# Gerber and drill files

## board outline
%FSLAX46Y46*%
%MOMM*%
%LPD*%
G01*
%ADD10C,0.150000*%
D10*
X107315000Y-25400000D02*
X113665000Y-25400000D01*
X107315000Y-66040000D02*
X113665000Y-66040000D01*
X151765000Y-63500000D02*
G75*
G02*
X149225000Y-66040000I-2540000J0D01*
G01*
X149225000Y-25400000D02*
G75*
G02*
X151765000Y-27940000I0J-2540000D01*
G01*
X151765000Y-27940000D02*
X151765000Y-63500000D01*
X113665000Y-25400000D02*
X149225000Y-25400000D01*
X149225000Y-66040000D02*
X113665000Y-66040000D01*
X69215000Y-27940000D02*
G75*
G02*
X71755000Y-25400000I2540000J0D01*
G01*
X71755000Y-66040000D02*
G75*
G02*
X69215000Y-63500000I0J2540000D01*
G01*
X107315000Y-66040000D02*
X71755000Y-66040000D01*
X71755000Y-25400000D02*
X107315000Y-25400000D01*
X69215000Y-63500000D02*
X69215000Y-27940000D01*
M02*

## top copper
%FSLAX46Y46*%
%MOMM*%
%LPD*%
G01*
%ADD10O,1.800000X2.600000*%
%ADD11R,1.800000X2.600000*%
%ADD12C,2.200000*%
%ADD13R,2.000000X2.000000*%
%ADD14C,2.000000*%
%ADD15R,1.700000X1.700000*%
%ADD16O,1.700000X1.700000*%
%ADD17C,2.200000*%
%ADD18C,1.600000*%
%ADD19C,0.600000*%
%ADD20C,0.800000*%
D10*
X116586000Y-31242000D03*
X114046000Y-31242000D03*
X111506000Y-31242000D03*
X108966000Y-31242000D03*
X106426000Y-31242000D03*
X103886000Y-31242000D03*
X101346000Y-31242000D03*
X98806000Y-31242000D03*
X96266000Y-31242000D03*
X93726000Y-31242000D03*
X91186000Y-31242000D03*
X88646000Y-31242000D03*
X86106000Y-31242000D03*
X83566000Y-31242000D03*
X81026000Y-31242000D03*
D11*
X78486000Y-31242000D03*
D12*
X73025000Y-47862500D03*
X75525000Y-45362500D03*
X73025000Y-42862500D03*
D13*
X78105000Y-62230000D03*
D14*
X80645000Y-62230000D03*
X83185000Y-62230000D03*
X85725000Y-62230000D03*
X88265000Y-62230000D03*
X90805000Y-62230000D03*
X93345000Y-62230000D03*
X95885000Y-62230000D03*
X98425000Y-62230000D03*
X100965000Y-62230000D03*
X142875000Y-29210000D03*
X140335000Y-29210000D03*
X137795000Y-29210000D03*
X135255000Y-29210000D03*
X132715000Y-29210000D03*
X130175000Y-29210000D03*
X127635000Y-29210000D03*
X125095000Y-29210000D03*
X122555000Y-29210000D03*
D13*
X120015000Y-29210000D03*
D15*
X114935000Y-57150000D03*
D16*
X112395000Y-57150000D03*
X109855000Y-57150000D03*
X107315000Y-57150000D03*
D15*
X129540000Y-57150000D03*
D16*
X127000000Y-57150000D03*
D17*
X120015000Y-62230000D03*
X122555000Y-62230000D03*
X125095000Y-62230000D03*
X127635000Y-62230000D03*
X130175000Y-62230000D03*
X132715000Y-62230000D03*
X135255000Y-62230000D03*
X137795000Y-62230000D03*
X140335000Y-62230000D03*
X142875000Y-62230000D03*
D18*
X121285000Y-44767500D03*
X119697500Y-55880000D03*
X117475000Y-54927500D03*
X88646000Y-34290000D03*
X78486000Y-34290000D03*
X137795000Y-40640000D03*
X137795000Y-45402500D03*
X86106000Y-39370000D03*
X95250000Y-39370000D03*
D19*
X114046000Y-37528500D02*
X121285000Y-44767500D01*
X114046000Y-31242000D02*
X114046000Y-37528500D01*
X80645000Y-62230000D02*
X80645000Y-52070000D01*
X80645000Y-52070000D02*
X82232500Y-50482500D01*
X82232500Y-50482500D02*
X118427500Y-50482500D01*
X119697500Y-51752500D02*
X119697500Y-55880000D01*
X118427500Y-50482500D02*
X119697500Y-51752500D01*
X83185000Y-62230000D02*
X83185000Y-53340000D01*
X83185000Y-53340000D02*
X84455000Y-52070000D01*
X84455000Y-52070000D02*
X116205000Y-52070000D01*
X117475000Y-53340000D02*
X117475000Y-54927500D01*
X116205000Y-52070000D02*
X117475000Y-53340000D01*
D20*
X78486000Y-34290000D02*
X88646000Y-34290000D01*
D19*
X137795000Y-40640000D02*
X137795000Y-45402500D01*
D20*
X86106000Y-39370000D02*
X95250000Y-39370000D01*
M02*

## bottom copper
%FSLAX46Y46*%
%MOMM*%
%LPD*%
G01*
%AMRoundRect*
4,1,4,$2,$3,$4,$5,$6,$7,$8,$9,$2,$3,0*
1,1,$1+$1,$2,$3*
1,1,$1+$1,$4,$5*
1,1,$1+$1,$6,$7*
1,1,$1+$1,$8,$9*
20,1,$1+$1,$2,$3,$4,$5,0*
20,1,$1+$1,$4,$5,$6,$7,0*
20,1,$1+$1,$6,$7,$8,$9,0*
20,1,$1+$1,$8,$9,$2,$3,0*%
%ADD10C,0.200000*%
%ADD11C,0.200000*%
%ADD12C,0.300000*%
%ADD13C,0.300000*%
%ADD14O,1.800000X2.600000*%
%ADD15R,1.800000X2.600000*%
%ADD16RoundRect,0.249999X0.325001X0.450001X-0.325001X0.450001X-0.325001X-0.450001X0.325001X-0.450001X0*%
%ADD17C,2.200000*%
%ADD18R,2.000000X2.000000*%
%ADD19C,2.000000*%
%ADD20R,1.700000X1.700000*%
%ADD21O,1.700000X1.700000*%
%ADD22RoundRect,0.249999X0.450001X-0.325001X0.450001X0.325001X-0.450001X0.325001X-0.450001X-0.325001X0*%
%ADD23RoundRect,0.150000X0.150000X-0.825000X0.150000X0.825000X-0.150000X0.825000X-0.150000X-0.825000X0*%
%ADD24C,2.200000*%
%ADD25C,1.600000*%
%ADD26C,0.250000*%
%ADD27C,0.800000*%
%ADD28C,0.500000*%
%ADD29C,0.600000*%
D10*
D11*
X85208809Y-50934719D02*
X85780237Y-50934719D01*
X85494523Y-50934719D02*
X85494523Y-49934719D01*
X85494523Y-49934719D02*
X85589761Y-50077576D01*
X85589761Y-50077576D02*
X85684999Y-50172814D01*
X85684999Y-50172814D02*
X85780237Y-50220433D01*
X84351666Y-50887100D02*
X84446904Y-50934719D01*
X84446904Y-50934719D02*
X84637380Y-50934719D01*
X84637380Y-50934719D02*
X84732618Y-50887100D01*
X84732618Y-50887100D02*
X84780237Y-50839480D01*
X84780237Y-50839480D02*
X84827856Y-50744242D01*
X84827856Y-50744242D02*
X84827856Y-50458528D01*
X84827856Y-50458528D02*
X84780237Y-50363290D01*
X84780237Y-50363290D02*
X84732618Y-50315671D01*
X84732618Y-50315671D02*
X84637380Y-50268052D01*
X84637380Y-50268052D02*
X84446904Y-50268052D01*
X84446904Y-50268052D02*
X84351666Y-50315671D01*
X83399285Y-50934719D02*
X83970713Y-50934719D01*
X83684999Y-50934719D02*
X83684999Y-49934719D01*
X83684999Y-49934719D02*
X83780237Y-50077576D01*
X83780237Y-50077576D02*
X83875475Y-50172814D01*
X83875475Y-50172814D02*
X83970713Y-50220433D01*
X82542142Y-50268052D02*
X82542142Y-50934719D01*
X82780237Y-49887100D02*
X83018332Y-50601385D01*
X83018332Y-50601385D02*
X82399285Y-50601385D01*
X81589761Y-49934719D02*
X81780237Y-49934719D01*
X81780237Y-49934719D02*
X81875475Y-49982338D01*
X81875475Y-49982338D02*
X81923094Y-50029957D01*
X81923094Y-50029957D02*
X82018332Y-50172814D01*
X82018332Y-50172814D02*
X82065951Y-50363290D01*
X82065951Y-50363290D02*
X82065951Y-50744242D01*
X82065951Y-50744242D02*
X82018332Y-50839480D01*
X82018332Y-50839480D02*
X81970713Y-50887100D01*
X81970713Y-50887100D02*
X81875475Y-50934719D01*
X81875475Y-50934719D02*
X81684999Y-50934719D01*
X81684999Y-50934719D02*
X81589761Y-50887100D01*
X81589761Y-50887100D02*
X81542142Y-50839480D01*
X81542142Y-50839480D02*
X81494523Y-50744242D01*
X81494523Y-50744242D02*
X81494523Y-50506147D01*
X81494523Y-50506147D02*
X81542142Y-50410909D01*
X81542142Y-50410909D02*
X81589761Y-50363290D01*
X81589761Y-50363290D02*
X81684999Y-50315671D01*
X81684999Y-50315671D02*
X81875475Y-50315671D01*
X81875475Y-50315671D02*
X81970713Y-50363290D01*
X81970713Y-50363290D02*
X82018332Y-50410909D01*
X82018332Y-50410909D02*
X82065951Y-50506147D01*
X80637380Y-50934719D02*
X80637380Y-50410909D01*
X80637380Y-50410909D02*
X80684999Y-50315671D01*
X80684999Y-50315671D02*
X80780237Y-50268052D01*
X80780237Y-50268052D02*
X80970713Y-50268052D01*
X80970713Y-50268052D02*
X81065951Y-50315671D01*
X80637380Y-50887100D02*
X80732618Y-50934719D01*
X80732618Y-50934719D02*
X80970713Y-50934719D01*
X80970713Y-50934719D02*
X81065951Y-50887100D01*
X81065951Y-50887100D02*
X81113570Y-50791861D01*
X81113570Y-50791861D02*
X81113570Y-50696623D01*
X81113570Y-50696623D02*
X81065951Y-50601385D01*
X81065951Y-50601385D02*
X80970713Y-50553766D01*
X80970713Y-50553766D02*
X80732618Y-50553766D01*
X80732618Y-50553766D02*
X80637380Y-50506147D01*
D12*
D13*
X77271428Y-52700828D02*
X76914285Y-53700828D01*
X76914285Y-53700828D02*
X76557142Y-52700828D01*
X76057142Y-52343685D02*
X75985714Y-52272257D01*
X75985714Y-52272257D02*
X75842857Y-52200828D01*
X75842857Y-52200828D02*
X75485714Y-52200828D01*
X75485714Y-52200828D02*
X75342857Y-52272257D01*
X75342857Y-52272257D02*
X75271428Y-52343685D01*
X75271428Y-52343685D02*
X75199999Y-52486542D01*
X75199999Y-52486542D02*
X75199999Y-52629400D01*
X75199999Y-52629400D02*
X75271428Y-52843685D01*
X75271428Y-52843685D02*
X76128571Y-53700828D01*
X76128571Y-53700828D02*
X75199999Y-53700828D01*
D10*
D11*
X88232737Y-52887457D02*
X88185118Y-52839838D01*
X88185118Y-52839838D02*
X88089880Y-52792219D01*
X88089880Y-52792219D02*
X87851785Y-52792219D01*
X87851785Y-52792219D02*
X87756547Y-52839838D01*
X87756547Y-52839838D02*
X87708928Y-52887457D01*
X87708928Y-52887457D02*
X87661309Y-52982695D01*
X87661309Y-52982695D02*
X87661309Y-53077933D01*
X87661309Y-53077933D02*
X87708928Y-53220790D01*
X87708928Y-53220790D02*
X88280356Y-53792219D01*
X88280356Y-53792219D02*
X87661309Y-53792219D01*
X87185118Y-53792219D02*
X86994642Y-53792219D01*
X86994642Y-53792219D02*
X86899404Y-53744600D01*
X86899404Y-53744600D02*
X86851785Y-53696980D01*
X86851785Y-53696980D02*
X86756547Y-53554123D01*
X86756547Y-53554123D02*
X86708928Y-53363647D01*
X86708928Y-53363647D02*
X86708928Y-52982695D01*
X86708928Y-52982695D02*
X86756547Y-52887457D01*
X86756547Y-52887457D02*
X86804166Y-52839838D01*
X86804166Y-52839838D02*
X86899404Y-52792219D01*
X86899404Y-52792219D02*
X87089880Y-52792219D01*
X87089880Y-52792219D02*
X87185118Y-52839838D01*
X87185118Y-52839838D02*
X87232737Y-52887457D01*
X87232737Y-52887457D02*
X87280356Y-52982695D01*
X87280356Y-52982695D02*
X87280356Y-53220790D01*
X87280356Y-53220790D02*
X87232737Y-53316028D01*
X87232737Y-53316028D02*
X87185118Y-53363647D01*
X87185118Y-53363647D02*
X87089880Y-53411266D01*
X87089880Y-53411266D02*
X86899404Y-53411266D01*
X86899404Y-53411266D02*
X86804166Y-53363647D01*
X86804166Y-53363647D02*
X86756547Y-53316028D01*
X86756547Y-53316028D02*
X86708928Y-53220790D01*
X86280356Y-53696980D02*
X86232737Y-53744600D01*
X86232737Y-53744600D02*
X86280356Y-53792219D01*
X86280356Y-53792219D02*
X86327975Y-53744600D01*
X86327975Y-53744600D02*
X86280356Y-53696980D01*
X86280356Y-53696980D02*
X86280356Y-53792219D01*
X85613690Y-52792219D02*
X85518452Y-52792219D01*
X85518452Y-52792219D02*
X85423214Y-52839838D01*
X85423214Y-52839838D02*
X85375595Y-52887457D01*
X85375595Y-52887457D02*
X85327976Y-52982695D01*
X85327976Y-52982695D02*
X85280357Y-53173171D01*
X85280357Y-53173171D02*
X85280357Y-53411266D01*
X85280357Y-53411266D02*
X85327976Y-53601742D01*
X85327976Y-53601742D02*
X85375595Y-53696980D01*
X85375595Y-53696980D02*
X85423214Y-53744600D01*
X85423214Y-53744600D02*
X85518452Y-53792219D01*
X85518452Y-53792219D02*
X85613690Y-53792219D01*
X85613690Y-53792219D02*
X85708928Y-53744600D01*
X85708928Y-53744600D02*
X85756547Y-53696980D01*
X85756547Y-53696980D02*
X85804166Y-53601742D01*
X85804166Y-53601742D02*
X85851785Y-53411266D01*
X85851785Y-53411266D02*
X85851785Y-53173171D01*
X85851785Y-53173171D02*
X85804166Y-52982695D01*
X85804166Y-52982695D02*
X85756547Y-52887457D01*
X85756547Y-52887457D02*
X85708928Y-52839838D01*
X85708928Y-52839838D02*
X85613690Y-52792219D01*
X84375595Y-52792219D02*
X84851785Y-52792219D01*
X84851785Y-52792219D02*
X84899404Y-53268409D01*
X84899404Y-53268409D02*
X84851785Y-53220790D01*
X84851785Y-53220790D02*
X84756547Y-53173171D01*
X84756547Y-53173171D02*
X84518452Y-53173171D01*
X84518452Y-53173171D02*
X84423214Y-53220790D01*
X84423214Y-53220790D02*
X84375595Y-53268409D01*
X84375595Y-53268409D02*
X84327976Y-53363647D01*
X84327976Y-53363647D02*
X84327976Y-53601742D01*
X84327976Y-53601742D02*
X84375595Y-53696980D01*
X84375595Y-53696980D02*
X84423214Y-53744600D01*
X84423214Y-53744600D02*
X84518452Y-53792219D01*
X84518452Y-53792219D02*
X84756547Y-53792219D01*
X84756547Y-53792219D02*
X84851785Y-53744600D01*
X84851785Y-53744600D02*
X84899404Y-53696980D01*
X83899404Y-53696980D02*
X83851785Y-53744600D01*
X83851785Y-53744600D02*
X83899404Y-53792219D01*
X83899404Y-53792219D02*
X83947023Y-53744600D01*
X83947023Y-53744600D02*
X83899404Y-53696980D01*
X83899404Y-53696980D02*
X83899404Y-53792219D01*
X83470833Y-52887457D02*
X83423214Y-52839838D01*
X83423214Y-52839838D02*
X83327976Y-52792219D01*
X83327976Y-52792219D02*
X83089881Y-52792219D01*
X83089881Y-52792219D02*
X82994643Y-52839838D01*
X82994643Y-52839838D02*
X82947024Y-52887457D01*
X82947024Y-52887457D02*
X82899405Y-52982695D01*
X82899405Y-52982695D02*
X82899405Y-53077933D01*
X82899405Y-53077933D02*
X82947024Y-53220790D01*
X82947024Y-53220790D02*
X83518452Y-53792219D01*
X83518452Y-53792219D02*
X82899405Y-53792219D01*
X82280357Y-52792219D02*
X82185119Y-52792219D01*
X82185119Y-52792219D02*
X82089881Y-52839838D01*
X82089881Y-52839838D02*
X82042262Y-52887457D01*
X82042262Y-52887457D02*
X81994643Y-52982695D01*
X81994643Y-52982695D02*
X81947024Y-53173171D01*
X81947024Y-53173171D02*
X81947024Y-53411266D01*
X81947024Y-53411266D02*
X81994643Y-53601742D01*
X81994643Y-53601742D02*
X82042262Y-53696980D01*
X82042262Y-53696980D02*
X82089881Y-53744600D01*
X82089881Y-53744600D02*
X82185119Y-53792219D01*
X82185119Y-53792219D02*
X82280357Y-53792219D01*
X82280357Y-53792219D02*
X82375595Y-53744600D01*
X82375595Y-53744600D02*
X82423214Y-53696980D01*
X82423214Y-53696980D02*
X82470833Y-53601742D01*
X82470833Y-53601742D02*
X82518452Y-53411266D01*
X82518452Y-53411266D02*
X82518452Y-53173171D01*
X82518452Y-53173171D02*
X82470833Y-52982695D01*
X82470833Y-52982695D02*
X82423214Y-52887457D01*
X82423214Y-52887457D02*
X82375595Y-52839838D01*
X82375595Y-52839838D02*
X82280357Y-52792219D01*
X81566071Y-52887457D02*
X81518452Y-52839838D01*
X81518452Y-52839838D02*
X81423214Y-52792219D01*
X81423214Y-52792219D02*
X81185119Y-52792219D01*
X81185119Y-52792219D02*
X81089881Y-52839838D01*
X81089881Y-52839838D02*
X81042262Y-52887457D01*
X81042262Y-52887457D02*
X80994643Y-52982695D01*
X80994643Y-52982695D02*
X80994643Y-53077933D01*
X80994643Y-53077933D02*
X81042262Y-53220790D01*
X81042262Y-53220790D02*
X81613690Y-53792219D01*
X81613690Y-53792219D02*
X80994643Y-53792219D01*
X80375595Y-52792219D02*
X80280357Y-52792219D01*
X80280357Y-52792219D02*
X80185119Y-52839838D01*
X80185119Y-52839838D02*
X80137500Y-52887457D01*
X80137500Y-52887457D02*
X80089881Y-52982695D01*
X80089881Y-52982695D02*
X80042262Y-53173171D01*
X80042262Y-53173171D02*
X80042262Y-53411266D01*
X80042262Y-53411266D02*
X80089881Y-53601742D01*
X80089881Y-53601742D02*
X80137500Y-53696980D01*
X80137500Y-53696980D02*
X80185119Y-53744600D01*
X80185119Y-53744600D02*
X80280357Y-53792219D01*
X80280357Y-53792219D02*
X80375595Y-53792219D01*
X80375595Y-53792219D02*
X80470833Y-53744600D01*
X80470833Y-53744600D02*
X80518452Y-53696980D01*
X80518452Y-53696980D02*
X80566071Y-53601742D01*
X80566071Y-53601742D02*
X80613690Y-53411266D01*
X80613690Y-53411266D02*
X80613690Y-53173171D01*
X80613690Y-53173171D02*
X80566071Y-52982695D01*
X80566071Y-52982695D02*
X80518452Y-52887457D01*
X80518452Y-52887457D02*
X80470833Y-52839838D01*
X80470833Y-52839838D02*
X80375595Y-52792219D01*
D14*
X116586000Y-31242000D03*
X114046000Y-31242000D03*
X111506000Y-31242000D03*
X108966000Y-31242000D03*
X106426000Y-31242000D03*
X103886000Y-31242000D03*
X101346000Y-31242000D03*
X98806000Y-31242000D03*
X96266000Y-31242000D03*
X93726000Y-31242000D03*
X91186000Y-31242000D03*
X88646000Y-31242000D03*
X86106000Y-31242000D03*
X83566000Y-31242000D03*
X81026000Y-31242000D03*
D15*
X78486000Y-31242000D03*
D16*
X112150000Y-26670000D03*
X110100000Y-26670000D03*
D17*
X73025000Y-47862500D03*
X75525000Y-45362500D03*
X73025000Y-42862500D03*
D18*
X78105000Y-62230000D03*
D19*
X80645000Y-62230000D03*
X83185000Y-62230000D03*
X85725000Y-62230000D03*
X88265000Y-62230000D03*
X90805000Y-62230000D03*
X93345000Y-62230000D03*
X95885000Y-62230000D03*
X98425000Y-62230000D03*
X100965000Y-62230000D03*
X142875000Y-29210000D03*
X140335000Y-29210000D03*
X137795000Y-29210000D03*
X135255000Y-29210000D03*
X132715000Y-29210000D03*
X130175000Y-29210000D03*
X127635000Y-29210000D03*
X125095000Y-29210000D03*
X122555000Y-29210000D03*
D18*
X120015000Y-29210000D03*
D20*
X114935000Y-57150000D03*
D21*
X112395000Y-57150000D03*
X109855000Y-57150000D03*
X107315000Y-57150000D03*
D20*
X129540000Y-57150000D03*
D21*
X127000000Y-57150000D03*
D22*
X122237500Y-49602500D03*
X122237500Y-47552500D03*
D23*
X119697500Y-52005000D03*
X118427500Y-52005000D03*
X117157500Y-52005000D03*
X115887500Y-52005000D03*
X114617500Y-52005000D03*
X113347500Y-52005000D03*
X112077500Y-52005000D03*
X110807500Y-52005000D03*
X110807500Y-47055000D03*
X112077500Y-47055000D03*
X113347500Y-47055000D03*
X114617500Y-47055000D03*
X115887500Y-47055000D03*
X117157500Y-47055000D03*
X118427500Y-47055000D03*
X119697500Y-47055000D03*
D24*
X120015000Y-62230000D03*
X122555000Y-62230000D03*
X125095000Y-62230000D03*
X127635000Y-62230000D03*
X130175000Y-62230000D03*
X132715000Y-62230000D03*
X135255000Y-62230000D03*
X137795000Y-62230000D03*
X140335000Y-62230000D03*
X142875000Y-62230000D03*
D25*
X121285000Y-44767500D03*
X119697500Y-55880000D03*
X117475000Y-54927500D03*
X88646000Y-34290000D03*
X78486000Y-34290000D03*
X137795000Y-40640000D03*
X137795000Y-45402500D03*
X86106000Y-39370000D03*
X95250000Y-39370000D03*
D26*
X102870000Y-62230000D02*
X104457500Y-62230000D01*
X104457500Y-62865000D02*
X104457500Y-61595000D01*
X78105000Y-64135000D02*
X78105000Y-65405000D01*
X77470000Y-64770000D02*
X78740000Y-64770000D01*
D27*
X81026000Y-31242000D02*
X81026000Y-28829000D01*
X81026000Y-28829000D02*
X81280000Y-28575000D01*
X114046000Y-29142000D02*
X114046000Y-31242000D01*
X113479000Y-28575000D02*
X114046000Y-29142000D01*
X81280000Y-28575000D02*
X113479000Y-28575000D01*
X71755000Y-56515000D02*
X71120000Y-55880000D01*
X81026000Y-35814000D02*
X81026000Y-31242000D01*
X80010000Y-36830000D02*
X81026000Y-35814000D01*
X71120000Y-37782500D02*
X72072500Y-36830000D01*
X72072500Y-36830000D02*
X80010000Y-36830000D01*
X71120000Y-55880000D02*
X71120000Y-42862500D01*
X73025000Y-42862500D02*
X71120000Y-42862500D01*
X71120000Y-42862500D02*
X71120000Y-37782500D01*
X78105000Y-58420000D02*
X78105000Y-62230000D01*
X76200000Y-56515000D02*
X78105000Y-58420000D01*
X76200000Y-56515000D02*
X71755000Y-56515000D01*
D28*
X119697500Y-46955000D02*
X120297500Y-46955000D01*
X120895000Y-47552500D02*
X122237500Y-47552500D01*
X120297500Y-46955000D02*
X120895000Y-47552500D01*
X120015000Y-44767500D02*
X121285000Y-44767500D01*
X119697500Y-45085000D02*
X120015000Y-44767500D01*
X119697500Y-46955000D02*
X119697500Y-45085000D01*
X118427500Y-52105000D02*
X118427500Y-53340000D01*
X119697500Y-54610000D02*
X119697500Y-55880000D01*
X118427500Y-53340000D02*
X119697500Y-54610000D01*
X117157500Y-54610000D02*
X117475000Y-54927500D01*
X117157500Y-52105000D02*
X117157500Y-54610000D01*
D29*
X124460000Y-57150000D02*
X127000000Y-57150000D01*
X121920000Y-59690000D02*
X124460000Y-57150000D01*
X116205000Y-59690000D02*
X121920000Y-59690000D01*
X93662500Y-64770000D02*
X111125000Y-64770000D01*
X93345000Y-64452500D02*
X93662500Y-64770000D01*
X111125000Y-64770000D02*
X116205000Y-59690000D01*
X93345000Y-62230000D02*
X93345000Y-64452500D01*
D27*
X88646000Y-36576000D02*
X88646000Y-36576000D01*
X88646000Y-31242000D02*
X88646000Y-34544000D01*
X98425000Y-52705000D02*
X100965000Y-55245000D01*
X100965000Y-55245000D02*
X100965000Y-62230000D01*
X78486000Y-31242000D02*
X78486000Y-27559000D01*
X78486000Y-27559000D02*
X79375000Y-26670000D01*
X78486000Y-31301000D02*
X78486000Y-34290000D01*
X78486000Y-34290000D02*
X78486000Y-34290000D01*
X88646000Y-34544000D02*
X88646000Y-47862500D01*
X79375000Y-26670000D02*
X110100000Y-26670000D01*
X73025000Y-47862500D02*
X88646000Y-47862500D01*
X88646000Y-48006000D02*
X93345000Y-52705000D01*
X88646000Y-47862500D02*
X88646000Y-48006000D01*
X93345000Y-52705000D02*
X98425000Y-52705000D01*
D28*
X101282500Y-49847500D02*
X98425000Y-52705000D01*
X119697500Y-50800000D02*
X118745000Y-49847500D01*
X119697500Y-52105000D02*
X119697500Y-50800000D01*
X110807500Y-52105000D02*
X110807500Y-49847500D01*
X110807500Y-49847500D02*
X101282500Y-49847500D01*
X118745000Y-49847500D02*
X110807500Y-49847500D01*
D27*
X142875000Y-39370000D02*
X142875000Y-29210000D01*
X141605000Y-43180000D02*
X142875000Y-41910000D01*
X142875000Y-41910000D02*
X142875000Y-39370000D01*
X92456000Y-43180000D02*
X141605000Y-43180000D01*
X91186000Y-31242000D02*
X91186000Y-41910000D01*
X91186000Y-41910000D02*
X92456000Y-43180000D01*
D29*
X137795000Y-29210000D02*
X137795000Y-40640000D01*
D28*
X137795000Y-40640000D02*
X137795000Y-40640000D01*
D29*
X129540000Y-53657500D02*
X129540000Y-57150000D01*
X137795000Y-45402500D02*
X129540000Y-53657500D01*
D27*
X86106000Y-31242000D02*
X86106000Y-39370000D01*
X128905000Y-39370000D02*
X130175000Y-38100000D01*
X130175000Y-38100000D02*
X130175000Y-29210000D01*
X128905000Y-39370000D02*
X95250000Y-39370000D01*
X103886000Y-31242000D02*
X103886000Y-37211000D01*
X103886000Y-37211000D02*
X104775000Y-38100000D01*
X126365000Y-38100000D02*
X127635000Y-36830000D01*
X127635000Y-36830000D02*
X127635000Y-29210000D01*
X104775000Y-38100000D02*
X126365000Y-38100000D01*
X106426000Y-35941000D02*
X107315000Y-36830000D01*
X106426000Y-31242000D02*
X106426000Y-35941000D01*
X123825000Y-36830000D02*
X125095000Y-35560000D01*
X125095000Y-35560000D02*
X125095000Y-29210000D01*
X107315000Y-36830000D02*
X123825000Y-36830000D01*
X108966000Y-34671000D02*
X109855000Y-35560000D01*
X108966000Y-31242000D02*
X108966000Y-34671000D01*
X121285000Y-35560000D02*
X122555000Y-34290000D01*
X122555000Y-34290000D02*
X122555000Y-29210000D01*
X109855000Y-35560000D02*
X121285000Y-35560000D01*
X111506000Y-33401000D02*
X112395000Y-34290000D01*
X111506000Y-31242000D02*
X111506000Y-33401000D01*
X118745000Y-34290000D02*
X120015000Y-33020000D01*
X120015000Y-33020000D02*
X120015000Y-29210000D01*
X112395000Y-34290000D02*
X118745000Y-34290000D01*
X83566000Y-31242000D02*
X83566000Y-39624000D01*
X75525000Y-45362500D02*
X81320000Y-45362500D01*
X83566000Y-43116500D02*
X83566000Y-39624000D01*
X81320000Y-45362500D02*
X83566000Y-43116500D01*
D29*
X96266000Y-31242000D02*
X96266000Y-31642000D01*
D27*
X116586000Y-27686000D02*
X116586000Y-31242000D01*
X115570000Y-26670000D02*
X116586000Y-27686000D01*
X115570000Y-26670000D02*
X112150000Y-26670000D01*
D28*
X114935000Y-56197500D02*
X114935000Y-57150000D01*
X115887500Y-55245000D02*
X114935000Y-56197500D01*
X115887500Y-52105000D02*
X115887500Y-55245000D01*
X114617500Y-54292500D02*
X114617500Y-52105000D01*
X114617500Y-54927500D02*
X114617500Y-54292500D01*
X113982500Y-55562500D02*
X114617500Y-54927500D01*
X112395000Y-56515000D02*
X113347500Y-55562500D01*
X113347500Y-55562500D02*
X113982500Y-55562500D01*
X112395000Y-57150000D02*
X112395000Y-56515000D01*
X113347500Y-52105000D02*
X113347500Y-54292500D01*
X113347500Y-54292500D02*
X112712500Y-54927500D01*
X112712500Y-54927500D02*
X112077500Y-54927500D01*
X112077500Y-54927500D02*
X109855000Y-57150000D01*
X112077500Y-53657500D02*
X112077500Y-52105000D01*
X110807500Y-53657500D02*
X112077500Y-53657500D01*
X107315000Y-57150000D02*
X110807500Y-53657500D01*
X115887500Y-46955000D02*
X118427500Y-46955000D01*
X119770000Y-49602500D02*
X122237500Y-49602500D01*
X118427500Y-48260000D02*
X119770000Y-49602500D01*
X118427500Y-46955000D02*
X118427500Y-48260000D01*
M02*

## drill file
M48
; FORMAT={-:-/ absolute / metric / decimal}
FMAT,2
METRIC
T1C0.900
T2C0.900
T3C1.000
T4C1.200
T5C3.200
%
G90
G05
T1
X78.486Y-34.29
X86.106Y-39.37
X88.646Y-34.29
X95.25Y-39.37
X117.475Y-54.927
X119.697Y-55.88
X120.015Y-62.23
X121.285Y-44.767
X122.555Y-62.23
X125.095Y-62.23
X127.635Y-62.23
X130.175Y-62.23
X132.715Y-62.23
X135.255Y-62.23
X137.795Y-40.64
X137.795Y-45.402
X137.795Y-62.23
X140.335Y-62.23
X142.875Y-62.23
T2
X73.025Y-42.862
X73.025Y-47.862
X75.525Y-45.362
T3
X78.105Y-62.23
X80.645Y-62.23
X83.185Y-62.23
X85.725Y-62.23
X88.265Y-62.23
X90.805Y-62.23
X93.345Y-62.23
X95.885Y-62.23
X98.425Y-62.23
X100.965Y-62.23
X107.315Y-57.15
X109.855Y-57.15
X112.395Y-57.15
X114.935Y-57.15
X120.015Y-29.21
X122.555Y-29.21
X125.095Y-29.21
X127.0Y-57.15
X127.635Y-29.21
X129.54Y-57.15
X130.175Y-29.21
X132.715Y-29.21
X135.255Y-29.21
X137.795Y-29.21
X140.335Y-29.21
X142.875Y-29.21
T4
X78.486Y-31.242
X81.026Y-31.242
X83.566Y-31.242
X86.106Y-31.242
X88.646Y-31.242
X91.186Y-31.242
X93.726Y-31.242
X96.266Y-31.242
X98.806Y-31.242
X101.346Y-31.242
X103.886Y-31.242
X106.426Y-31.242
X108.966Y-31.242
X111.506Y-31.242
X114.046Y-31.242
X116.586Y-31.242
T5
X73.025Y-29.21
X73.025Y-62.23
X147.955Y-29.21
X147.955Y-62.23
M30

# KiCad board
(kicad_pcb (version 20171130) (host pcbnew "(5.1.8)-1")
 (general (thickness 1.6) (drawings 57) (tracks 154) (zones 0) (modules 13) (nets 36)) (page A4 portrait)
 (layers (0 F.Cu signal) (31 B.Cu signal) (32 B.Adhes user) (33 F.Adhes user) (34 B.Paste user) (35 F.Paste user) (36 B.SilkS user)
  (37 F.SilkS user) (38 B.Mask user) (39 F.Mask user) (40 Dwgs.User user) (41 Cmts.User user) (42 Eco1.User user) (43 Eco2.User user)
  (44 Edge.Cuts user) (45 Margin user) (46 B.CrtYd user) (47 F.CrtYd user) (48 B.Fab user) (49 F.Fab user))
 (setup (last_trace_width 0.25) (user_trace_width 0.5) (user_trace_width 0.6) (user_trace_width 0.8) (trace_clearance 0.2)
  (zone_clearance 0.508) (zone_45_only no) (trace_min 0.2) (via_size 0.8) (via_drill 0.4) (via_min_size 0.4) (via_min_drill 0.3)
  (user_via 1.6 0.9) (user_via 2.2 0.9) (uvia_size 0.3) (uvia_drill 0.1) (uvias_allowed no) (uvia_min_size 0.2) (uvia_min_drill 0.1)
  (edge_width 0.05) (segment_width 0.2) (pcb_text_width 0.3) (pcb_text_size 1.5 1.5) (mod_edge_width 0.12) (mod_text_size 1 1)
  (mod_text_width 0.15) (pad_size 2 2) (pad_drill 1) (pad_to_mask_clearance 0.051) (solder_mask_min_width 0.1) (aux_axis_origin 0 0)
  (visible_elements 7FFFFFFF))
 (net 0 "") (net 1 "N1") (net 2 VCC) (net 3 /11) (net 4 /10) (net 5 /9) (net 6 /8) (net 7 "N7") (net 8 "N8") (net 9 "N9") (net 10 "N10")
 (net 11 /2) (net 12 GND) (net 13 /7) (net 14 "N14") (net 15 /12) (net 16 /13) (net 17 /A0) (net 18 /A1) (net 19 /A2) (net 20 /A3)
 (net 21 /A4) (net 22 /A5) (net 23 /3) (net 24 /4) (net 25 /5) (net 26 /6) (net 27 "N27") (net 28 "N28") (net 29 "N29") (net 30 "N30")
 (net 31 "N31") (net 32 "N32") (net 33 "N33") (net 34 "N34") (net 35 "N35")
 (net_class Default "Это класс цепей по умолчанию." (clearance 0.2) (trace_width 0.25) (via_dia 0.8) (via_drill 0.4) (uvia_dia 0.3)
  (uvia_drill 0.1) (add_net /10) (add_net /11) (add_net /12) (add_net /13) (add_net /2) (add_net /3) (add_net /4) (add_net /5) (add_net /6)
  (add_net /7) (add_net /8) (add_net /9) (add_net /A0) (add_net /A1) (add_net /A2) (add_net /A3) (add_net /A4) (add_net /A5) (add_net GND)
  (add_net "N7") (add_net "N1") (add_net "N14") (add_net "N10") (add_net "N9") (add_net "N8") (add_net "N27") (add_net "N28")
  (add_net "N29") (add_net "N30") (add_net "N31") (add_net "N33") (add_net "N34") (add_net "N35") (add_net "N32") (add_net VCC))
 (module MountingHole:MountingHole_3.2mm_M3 (layer F.Cu) (at 147.955 62.23 90)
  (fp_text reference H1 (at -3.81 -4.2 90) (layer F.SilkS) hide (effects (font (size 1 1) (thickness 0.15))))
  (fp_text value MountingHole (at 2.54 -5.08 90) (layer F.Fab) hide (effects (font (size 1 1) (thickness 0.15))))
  (pad 1 np_thru_hole circle (at 0 0 90) (size 3.2 3.2) (drill 3.2) (layers *.Cu *.Mask)))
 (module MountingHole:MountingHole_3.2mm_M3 (layer F.Cu) (at 147.955 29.21 90)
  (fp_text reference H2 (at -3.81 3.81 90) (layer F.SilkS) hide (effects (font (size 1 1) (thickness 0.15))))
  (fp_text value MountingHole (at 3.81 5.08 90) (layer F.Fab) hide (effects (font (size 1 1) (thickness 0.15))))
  (pad 1 np_thru_hole circle (at 0 0 90) (size 3.2 3.2) (drill 3.2) (layers *.Cu *.Mask)))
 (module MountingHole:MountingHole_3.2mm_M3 (layer F.Cu) (at 73.025 62.23 90)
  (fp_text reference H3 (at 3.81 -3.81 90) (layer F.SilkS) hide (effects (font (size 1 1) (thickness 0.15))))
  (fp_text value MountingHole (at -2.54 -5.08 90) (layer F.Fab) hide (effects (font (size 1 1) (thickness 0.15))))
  (pad 1 np_thru_hole circle (at 0 0 90) (size 3.2 3.2) (drill 3.2) (layers *.Cu *.Mask)))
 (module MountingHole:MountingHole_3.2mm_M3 (layer F.Cu) (at 73.025 29.21 90)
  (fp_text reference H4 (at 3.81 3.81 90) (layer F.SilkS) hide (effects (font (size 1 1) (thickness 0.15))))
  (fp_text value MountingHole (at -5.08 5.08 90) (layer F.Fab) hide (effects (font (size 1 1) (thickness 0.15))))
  (pad 1 np_thru_hole circle (at 0 0 90) (size 3.2 3.2) (drill 3.2) (layers *.Cu *.Mask)))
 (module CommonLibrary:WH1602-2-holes (layer F.Cu) (at 78.486 31.242)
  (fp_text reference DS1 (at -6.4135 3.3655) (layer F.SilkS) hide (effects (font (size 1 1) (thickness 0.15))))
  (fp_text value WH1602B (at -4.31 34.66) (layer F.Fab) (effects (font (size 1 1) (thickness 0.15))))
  (pad 16 thru_hole oval (at 38.1 0) (size 1.8 2.6) (drill 1.2) (layers *.Cu *.Mask) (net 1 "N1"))
  (pad 15 thru_hole oval (at 35.56 0) (size 1.8 2.6) (drill 1.2) (layers *.Cu *.Mask) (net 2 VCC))
  (pad 14 thru_hole oval (at 33.02 0) (size 1.8 2.6) (drill 1.2) (layers *.Cu *.Mask) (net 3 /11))
  (pad 13 thru_hole oval (at 30.48 0) (size 1.8 2.6) (drill 1.2) (layers *.Cu *.Mask) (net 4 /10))
  (pad 12 thru_hole oval (at 27.94 0) (size 1.8 2.6) (drill 1.2) (layers *.Cu *.Mask) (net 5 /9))
  (pad 11 thru_hole oval (at 25.4 0) (size 1.8 2.6) (drill 1.2) (layers *.Cu *.Mask) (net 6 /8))
  (pad 10 thru_hole oval (at 22.86 0) (size 1.8 2.6) (drill 1.2) (layers *.Cu *.Mask) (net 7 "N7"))
  (pad 9 thru_hole oval (at 20.32 0) (size 1.8 2.6) (drill 1.2) (layers *.Cu *.Mask) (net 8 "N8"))
  (pad 8 thru_hole oval (at 17.78 0) (size 1.8 2.6) (drill 1.2) (layers *.Cu *.Mask) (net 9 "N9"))
  (pad 7 thru_hole oval (at 15.24 0) (size 1.8 2.6) (drill 1.2) (layers *.Cu *.Mask) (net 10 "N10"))
  (pad 6 thru_hole oval (at 12.7 0) (size 1.8 2.6) (drill 1.2) (layers *.Cu *.Mask) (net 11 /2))
  (pad 5 thru_hole oval (at 10.16 0) (size 1.8 2.6) (drill 1.2) (layers *.Cu *.Mask) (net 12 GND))
  (pad 4 thru_hole oval (at 7.62 0) (size 1.8 2.6) (drill 1.2) (layers *.Cu *.Mask) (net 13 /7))
  (pad 3 thru_hole oval (at 5.08 0) (size 1.8 2.6) (drill 1.2) (layers *.Cu *.Mask) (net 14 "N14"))
  (pad 2 thru_hole oval (at 2.54 0) (size 1.8 2.6) (drill 1.2) (layers *.Cu *.Mask) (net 2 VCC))
  (pad 1 thru_hole rect (at 0 0) (size 1.8 2.6) (drill 1.2) (layers *.Cu *.Mask) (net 12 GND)))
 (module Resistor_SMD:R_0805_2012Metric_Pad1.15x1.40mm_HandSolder (layer B.Cu) (at 111.125 26.67 180)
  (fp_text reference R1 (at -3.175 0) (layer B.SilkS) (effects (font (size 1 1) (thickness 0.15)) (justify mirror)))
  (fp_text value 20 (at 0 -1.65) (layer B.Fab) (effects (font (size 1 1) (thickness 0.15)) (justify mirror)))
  (pad 1 smd roundrect (at -1.025 0 180) (size 1.15 1.4) (layers B.Cu B.Paste B.Mask) (roundrect_rratio 0.2173904347826087) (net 1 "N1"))
  (pad 2 smd roundrect (at 1.025 0 180) (size 1.15 1.4) (layers B.Cu B.Paste B.Mask) (roundrect_rratio 0.2173904347826087) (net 12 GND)))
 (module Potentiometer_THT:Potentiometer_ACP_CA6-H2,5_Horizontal (layer F.Cu) (at 73.025 42.8625)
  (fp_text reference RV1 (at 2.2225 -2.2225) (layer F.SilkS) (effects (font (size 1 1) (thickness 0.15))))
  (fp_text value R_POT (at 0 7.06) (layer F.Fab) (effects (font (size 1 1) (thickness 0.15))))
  (pad 3 thru_hole circle (at 0 5) (size 2.2 2.2) (drill 0.9) (layers *.Cu *.Mask) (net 12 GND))
  (pad 2 thru_hole circle (at 2.5 2.5) (size 2.2 2.2) (drill 0.9) (layers *.Cu *.Mask) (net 14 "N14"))
  (pad 1 thru_hole circle (at 0 0) (size 2.2 2.2) (drill 0.9) (layers *.Cu *.Mask) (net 2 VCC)))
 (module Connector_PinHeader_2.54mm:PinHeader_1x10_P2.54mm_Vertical (layer B.Cu) (at 78.105 62.23 270)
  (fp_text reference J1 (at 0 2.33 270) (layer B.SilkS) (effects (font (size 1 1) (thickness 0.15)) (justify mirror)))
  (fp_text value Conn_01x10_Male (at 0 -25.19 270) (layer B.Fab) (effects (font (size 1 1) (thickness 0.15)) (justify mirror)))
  (pad 1 thru_hole rect (at 0 0 270) (size 2 2) (drill 1) (layers *.Cu *.Mask) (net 2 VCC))
  (pad 2 thru_hole circle (at 0 -2.54 270) (size 2 2) (drill 1) (layers *.Cu *.Mask) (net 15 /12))
  (pad 3 thru_hole circle (at 0 -5.08 270) (size 2 2) (drill 1) (layers *.Cu *.Mask) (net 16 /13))
  (pad 4 thru_hole circle (at 0 -7.62 270) (size 2 2) (drill 1) (layers *.Cu *.Mask) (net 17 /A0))
  (pad 5 thru_hole circle (at 0 -10.16 270) (size 2 2) (drill 1) (layers *.Cu *.Mask) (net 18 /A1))
  (pad 6 thru_hole circle (at 0 -12.7 270) (size 2 2) (drill 1) (layers *.Cu *.Mask) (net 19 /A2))
  (pad 7 thru_hole circle (at 0 -15.24 270) (size 2 2) (drill 1) (layers *.Cu *.Mask) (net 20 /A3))
  (pad 8 thru_hole circle (at 0 -17.78 270) (size 2 2) (drill 1) (layers *.Cu *.Mask) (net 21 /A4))
  (pad 9 thru_hole circle (at 0 -20.32 270) (size 2 2) (drill 1) (layers *.Cu *.Mask) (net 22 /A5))
  (pad 10 thru_hole circle (at 0 -22.86 270) (size 2 2) (drill 1) (layers *.Cu *.Mask) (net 12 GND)))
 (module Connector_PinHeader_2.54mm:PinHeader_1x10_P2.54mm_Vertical (layer B.Cu) (at 120.015 29.21 270)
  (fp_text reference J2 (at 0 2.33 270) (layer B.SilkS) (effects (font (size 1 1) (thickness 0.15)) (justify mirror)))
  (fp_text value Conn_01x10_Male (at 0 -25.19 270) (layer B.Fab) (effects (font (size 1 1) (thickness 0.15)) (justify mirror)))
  (pad 10 thru_hole circle (at 0 -22.86 270) (size 2 2) (drill 1) (layers *.Cu *.Mask) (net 11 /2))
  (pad 9 thru_hole circle (at 0 -20.32 270) (size 2 2) (drill 1) (layers *.Cu *.Mask) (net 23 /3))
  (pad 8 thru_hole circle (at 0 -17.78 270) (size 2 2) (drill 1) (layers *.Cu *.Mask) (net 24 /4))
  (pad 7 thru_hole circle (at 0 -15.24 270) (size 2 2) (drill 1) (layers *.Cu *.Mask) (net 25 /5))
  (pad 6 thru_hole circle (at 0 -12.7 270) (size 2 2) (drill 1) (layers *.Cu *.Mask) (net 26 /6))
  (pad 5 thru_hole circle (at 0 -10.16 270) (size 2 2) (drill 1) (layers *.Cu *.Mask) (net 13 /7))
  (pad 4 thru_hole circle (at 0 -7.62 270) (size 2 2) (drill 1) (layers *.Cu *.Mask) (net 6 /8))
  (pad 3 thru_hole circle (at 0 -5.08 270) (size 2 2) (drill 1) (layers *.Cu *.Mask) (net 5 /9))
  (pad 2 thru_hole circle (at 0 -2.54 270) (size 2 2) (drill 1) (layers *.Cu *.Mask) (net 4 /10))
  (pad 1 thru_hole rect (at 0 0 270) (size 2 2) (drill 1) (layers *.Cu *.Mask) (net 3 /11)))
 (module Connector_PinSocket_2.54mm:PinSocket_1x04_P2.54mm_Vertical (layer F.Cu) (at 114.935 57.15 270)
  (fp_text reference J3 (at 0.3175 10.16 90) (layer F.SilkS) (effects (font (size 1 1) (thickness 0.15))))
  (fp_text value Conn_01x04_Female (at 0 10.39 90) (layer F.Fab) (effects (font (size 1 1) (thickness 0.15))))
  (pad 1 thru_hole rect (at 0 0 270) (size 1.7 1.7) (drill 1) (layers *.Cu *.Mask) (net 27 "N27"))
  (pad 2 thru_hole oval (at 0 2.54 270) (size 1.7 1.7) (drill 1) (layers *.Cu *.Mask) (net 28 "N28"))
  (pad 3 thru_hole oval (at 0 5.08 270) (size 1.7 1.7) (drill 1) (layers *.Cu *.Mask) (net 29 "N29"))
  (pad 4 thru_hole oval (at 0 7.62 270) (size 1.7 1.7) (drill 1) (layers *.Cu *.Mask) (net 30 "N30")))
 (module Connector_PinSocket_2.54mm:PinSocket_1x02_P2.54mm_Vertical (layer F.Cu) (at 129.54 57.15 270)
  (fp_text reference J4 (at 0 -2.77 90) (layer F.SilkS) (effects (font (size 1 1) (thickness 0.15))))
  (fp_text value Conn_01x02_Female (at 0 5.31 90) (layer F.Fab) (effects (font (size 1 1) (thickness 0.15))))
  (pad 1 thru_hole rect (at 0 0 270) (size 1.7 1.7) (drill 1) (layers *.Cu *.Mask) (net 24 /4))
  (pad 2 thru_hole oval (at 0 2.54 270) (size 1.7 1.7) (drill 1) (layers *.Cu *.Mask) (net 20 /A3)))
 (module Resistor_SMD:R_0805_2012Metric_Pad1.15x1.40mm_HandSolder (layer B.Cu) (at 122.2375 48.5775 90)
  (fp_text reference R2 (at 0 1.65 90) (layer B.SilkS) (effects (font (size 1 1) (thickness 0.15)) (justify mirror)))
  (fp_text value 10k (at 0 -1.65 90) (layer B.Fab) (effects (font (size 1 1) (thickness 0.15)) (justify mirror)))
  (pad 1 smd roundrect (at -1.025 0 90) (size 1.15 1.4) (layers B.Cu B.Paste B.Mask) (roundrect_rratio 0.2173904347826087) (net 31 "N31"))
  (pad 2 smd roundrect (at 1.025 0 90) (size 1.15 1.4) (layers B.Cu B.Paste B.Mask) (roundrect_rratio 0.2173904347826087) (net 2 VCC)))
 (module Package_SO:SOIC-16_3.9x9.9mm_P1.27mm (layer B.Cu) (at 115.2525 49.53 90)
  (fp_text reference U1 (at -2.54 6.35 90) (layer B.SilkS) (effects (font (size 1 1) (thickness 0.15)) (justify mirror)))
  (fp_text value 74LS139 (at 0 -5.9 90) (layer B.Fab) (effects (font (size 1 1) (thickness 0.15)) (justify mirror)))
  (pad 1 smd roundrect (at -2.475 4.445 90) (size 1.95 0.6) (layers B.Cu B.Paste B.Mask) (roundrect_rratio 0.25) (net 12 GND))
  (pad 2 smd roundrect (at -2.475 3.175 90) (size 1.95 0.6) (layers B.Cu B.Paste B.Mask) (roundrect_rratio 0.25) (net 15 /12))
  (pad 3 smd roundrect (at -2.475 1.905 90) (size 1.95 0.6) (layers B.Cu B.Paste B.Mask) (roundrect_rratio 0.25) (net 16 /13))
  (pad 4 smd roundrect (at -2.475 0.635 90) (size 1.95 0.6) (layers B.Cu B.Paste B.Mask) (roundrect_rratio 0.25) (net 27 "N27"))
  (pad 5 smd roundrect (at -2.475 -0.635 90) (size 1.95 0.6) (layers B.Cu B.Paste B.Mask) (roundrect_rratio 0.25) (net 28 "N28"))
  (pad 6 smd roundrect (at -2.475 -1.905 90) (size 1.95 0.6) (layers B.Cu B.Paste B.Mask) (roundrect_rratio 0.25) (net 29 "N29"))
  (pad 7 smd roundrect (at -2.475 -3.175 90) (size 1.95 0.6) (layers B.Cu B.Paste B.Mask) (roundrect_rratio 0.25) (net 30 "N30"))
  (pad 8 smd roundrect (at -2.475 -4.445 90) (size 1.95 0.6) (layers B.Cu B.Paste B.Mask) (roundrect_rratio 0.25) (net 12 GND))
  (pad 9 smd roundrect (at 2.475 -4.445 90) (size 1.95 0.6) (layers B.Cu B.Paste B.Mask) (roundrect_rratio 0.25) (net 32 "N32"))
  (pad 10 smd roundrect (at 2.475 -3.175 90) (size 1.95 0.6) (layers B.Cu B.Paste B.Mask) (roundrect_rratio 0.25) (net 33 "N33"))
  (pad 11 smd roundrect (at 2.475 -1.905 90) (size 1.95 0.6) (layers B.Cu B.Paste B.Mask) (roundrect_rratio 0.25) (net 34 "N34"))
  (pad 12 smd roundrect (at 2.475 -0.635 90) (size 1.95 0.6) (layers B.Cu B.Paste B.Mask) (roundrect_rratio 0.25) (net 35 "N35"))
  (pad 13 smd roundrect (at 2.475 0.635 90) (size 1.95 0.6) (layers B.Cu B.Paste B.Mask) (roundrect_rratio 0.25) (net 31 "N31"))
  (pad 14 smd roundrect (at 2.475 1.905 90) (size 1.95 0.6) (layers B.Cu B.Paste B.Mask) (roundrect_rratio 0.25) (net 31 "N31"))
  (pad 15 smd roundrect (at 2.475 3.175 90) (size 1.95 0.6) (layers B.Cu B.Paste B.Mask) (roundrect_rratio 0.25) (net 31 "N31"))
  (pad 16 smd roundrect (at 2.475 4.445 90) (size 1.95 0.6) (layers B.Cu B.Paste B.Mask) (roundrect_rratio 0.25) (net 2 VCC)))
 (gr_line (start 107.315 25.4) (end 113.665 25.4) (layer Edge.Cuts) (width 0.15))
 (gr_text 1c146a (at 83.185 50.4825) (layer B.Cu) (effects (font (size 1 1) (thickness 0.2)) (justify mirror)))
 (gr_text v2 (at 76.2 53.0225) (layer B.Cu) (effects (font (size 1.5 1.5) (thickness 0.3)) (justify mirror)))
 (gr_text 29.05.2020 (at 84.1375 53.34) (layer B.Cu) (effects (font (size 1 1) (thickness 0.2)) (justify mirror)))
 (gr_line (start 107.315 66.04) (end 113.665 66.04) (layer Edge.Cuts) (width 0.15))
 (gr_arc (start 149.225 63.5) (end 149.225 66.04) (angle -90) (layer Edge.Cuts) (width 0.15))
 (gr_arc (start 149.225 27.94) (end 151.765 27.94) (angle -90) (layer Edge.Cuts) (width 0.15))
 (gr_line (start 151.765 27.94) (end 151.765 63.5) (layer Edge.Cuts) (width 0.15))
 (gr_line (start 113.665 25.4) (end 149.225 25.4) (layer Edge.Cuts) (width 0.15))
 (gr_line (start 149.225 66.04) (end 113.665 66.04) (layer Edge.Cuts) (width 0.15))
 (gr_arc (start 71.755 27.94) (end 71.755 25.4) (angle -90) (layer Edge.Cuts) (width 0.15))
 (gr_arc (start 71.755 63.5) (end 69.215 63.5) (angle -90) (layer Edge.Cuts) (width 0.15))
 (gr_line (start 107.315 66.04) (end 71.755 66.04) (layer Edge.Cuts) (width 0.15))
 (gr_line (start 71.755 25.4) (end 107.315 25.4) (layer Edge.Cuts) (width 0.15))
 (gr_line (start 69.215 63.5) (end 69.215 27.94) (layer Edge.Cuts) (width 0.15))
 (segment (start 102.87 62.23) (end 104.4575 62.23) (width 0.25) (layer B.Cu) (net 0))
 (segment (start 104.4575 62.865) (end 104.4575 61.595) (width 0.25) (layer B.Cu) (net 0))
 (segment (start 78.105 64.135) (end 78.105 65.405) (width 0.25) (layer B.Cu) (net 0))
 (segment (start 77.47 64.77) (end 78.74 64.77) (width 0.25) (layer B.Cu) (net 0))
 (via (at 120.015 62.23) (size 2.2) (drill 0.9) (layers F.Cu B.Cu) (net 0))
 (via (at 122.555 62.23) (size 2.2) (drill 0.9) (layers F.Cu B.Cu) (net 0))
 (via (at 125.095 62.23) (size 2.2) (drill 0.9) (layers F.Cu B.Cu) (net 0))
 (via (at 127.635 62.23) (size 2.2) (drill 0.9) (layers F.Cu B.Cu) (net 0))
 (via (at 130.175 62.23) (size 2.2) (drill 0.9) (layers F.Cu B.Cu) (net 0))
 (via (at 132.715 62.23) (size 2.2) (drill 0.9) (layers F.Cu B.Cu) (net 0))
 (via (at 135.255 62.23) (size 2.2) (drill 0.9) (layers F.Cu B.Cu) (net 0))
 (via (at 137.795 62.23) (size 2.2) (drill 0.9) (layers F.Cu B.Cu) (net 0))
 (via (at 140.335 62.23) (size 2.2) (drill 0.9) (layers F.Cu B.Cu) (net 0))
 (via (at 142.875 62.23) (size 2.2) (drill 0.9) (layers F.Cu B.Cu) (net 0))
 (via (at 121.285 44.7675) (size 1.6) (drill 0.9) (layers F.Cu B.Cu) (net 2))
 (segment (start 81.026 31.242) (end 81.026 28.829) (width 0.8) (layer B.Cu) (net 2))
 (segment (start 81.026 28.829) (end 81.28 28.575) (width 0.8) (layer B.Cu) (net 2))
 (segment (start 114.046 29.142) (end 114.046 31.242) (width 0.8) (layer B.Cu) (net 2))
 (segment (start 113.479 28.575) (end 114.046 29.142) (width 0.8) (layer B.Cu) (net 2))
 (segment (start 81.28 28.575) (end 113.479 28.575) (width 0.8) (layer B.Cu) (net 2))
 (segment (start 71.755 56.515) (end 71.12 55.88) (width 0.8) (layer B.Cu) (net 2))
 (segment (start 81.026 35.814) (end 81.026 31.242) (width 0.8) (layer B.Cu) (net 2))
 (segment (start 80.01 36.83) (end 81.026 35.814) (width 0.8) (layer B.Cu) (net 2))
 (segment (start 71.12 37.7825) (end 72.0725 36.83) (width 0.8) (layer B.Cu) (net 2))
 (segment (start 72.0725 36.83) (end 80.01 36.83) (width 0.8) (layer B.Cu) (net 2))
 (segment (start 71.12 55.88) (end 71.12 42.8625) (width 0.8) (layer B.Cu) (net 2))
 (segment (start 73.025 42.8625) (end 71.12 42.8625) (width 0.8) (layer B.Cu) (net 2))
 (segment (start 71.12 42.8625) (end 71.12 37.7825) (width 0.8) (layer B.Cu) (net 2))
 (segment (start 78.105 58.42) (end 78.105 62.23) (width 0.8) (layer B.Cu) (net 2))
 (segment (start 76.2 56.515) (end 78.105 58.42) (width 0.8) (layer B.Cu) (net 2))
 (segment (start 76.2 56.515) (end 71.755 56.515) (width 0.8) (layer B.Cu) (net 2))
 (segment (start 119.6975 46.955) (end 120.2975 46.955) (width 0.5) (layer B.Cu) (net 2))
 (segment (start 120.895 47.5525) (end 122.2375 47.5525) (width 0.5) (layer B.Cu) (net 2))
 (segment (start 120.2975 46.955) (end 120.895 47.5525) (width 0.5) (layer B.Cu) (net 2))
 (segment (start 120.015 44.7675) (end 121.285 44.7675) (width 0.5) (layer B.Cu) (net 2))
 (segment (start 119.6975 45.085) (end 120.015 44.7675) (width 0.5) (layer B.Cu) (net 2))
 (segment (start 119.6975 46.955) (end 119.6975 45.085) (width 0.5) (layer B.Cu) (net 2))
 (segment (start 114.046 37.5285) (end 121.285 44.7675) (width 0.6) (layer F.Cu) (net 2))
 (segment (start 114.046 31.242) (end 114.046 37.5285) (width 0.6) (layer F.Cu) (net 2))
 (via (at 119.6975 55.88) (size 1.6) (drill 0.9) (layers F.Cu B.Cu) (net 15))
 (segment (start 118.4275 52.105) (end 118.4275 53.34) (width 0.5) (layer B.Cu) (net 15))
 (segment (start 119.6975 54.61) (end 119.6975 55.88) (width 0.5) (layer B.Cu) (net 15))
 (segment (start 118.4275 53.34) (end 119.6975 54.61) (width 0.5) (layer B.Cu) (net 15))
 (segment (start 80.645 62.23) (end 80.645 52.07) (width 0.6) (layer F.Cu) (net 15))
 (segment (start 80.645 52.07) (end 82.2325 50.4825) (width 0.6) (layer F.Cu) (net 15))
 (segment (start 82.2325 50.4825) (end 118.4275 50.4825) (width 0.6) (layer F.Cu) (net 15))
 (segment (start 119.6975 51.7525) (end 119.6975 55.88) (width 0.6) (layer F.Cu) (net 15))
 (segment (start 118.4275 50.4825) (end 119.6975 51.7525) (width 0.6) (layer F.Cu) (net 15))
 (via (at 117.475 54.9275) (size 1.6) (drill 0.9) (layers F.Cu B.Cu) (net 16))
 (segment (start 117.1575 54.61) (end 117.475 54.9275) (width 0.5) (layer B.Cu) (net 16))
 (segment (start 117.1575 52.105) (end 117.1575 54.61) (width 0.5) (layer B.Cu) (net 16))
 (segment (start 83.185 62.23) (end 83.185 53.34) (width 0.6) (layer F.Cu) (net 16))
 (segment (start 83.185 53.34) (end 84.455 52.07) (width 0.6) (layer F.Cu) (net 16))
 (segment (start 84.455 52.07) (end 116.205 52.07) (width 0.6) (layer F.Cu) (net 16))
 (segment (start 117.475 53.34) (end 117.475 54.9275) (width 0.6) (layer F.Cu) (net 16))
 (segment (start 116.205 52.07) (end 117.475 53.34) (width 0.6) (layer F.Cu) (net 16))
 (segment (start 124.46 57.15) (end 127 57.15) (width 0.6) (layer B.Cu) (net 20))
 (segment (start 121.92 59.69) (end 124.46 57.15) (width 0.6) (layer B.Cu) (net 20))
 (segment (start 116.205 59.69) (end 121.92 59.69) (width 0.6) (layer B.Cu) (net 20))
 (segment (start 93.6625 64.77) (end 111.125 64.77) (width 0.6) (layer B.Cu) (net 20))
 (segment (start 93.345 64.4525) (end 93.6625 64.77) (width 0.6) (layer B.Cu) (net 20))
 (segment (start 111.125 64.77) (end 116.205 59.69) (width 0.6) (layer B.Cu) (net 20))
 (segment (start 93.345 62.23) (end 93.345 64.4525) (width 0.6) (layer B.Cu) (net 20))
 (segment (start 88.646 36.576) (end 88.646 36.576) (width 0.8) (layer B.Cu) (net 12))
 (segment (start 88.646 31.242) (end 88.646 34.544) (width 0.8) (layer B.Cu) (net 12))
 (segment (start 98.425 52.705) (end 100.965 55.245) (width 0.8) (layer B.Cu) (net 12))
 (segment (start 100.965 55.245) (end 100.965 62.23) (width 0.8) (layer B.Cu) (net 12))
 (segment (start 78.486 31.242) (end 78.486 27.559) (width 0.8) (layer B.Cu) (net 12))
 (segment (start 78.486 27.559) (end 79.375 26.67) (width 0.8) (layer B.Cu) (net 12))
 (via (at 88.646 34.29) (size 1.6) (drill 0.9) (layers F.Cu B.Cu) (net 12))
 (segment (start 78.486 31.301) (end 78.486 34.29) (width 0.8) (layer B.Cu) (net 12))
 (segment (start 78.486 34.29) (end 78.486 34.29) (width 0.8) (layer B.Cu) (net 12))
 (via (at 78.486 34.29) (size 1.6) (drill 0.9) (layers F.Cu B.Cu) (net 12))
 (segment (start 78.486 34.29) (end 88.646 34.29) (width 0.8) (layer F.Cu) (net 12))
 (segment (start 88.646 34.544) (end 88.646 47.8625) (width 0.8) (layer B.Cu) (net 12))
 (segment (start 79.375 26.67) (end 110.1 26.67) (width 0.8) (layer B.Cu) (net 12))
 (segment (start 73.025 47.8625) (end 88.646 47.8625) (width 0.8) (layer B.Cu) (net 12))
 (segment (start 88.646 48.006) (end 93.345 52.705) (width 0.8) (layer B.Cu) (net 12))
 (segment (start 88.646 47.8625) (end 88.646 48.006) (width 0.8) (layer B.Cu) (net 12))
 (segment (start 93.345 52.705) (end 98.425 52.705) (width 0.8) (layer B.Cu) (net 12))
 (segment (start 101.2825 49.8475) (end 98.425 52.705) (width 0.5) (layer B.Cu) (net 12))
 (segment (start 119.6975 50.8) (end 118.745 49.8475) (width 0.5) (layer B.Cu) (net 12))
 (segment (start 119.6975 52.105) (end 119.6975 50.8) (width 0.5) (layer B.Cu) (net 12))
 (segment (start 110.8075 52.105) (end 110.8075 49.8475) (width 0.5) (layer B.Cu) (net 12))
 (segment (start 110.8075 49.8475) (end 101.2825 49.8475) (width 0.5) (layer B.Cu) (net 12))
 (segment (start 118.745 49.8475) (end 110.8075 49.8475) (width 0.5) (layer B.Cu) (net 12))
 (segment (start 142.875 39.37) (end 142.875 29.21) (width 0.8) (layer B.Cu) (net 11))
 (segment (start 141.605 43.18) (end 142.875 41.91) (width 0.8) (layer B.Cu) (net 11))
 (segment (start 142.875 41.91) (end 142.875 39.37) (width 0.8) (layer B.Cu) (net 11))
 (segment (start 92.456 43.18) (end 141.605 43.18) (width 0.8) (layer B.Cu) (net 11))
 (segment (start 91.186 31.242) (end 91.186 41.91) (width 0.8) (layer B.Cu) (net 11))
 (segment (start 91.186 41.91) (end 92.456 43.18) (width 0.8) (layer B.Cu) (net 11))
 (segment (start 137.795 29.21) (end 137.795 40.64) (width 0.6) (layer B.Cu) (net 24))
 (segment (start 137.795 40.64) (end 137.795 40.64) (width 0.5) (layer B.Cu) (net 24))
 (via (at 137.795 40.64) (size 1.6) (drill 0.9) (layers F.Cu B.Cu) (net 24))
 (segment (start 137.795 40.64) (end 137.795 45.4025) (width 0.6) (layer F.Cu) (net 24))
 (via (at 137.795 45.4025) (size 1.6) (drill 0.9) (layers F.Cu B.Cu) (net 24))
 (segment (start 129.54 53.6575) (end 129.54 57.15) (width 0.6) (layer B.Cu) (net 24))
 (segment (start 137.795 45.4025) (end 129.54 53.6575) (width 0.6) (layer B.Cu) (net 24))
 (segment (start 86.106 31.242) (end 86.106 39.37) (width 0.8) (layer B.Cu) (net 13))
 (segment (start 128.905 39.37) (end 130.175 38.1) (width 0.8) (layer B.Cu) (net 13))
 (segment (start 130.175 38.1) (end 130.175 29.21) (width 0.8) (layer B.Cu) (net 13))
 (segment (start 128.905 39.37) (end 95.25 39.37) (width 0.8) (layer B.Cu) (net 13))
 (via (at 86.106 39.37) (size 1.6) (drill 0.9) (layers F.Cu B.Cu) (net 13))
 (via (at 95.25 39.37) (size 1.6) (drill 0.9) (layers F.Cu B.Cu) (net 13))
 (segment (start 86.106 39.37) (end 95.25 39.37) (width 0.8) (layer F.Cu) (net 13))
 (segment (start 103.886 31.242) (end 103.886 37.211) (width 0.8) (layer B.Cu) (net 6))
 (segment (start 103.886 37.211) (end 104.775 38.1) (width 0.8) (layer B.Cu) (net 6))
 (segment (start 126.365 38.1) (end 127.635 36.83) (width 0.8) (layer B.Cu) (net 6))
 (segment (start 127.635 36.83) (end 127.635 29.21) (width 0.8) (layer B.Cu) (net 6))
 (segment (start 104.775 38.1) (end 126.365 38.1) (width 0.8) (layer B.Cu) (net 6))
 (segment (start 106.426 35.941) (end 107.315 36.83) (width 0.8) (layer B.Cu) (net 5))
 (segment (start 106.426 31.242) (end 106.426 35.941) (width 0.8) (layer B.Cu) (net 5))
 (segment (start 123.825 36.83) (end 125.095 35.56) (width 0.8) (layer B.Cu) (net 5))
 (segment (start 125.095 35.56) (end 125.095 29.21) (width 0.8) (layer B.Cu) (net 5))
 (segment (start 107.315 36.83) (end 123.825 36.83) (width 0.8) (layer B.Cu) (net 5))
 (segment (start 108.966 34.671) (end 109.855 35.56) (width 0.8) (layer B.Cu) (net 4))
 (segment (start 108.966 31.242) (end 108.966 34.671) (width 0.8) (layer B.Cu) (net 4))
 (segment (start 121.285 35.56) (end 122.555 34.29) (width 0.8) (layer B.Cu) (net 4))
 (segment (start 122.555 34.29) (end 122.555 29.21) (width 0.8) (layer B.Cu) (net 4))
 (segment (start 109.855 35.56) (end 121.285 35.56) (width 0.8) (layer B.Cu) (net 4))
 (segment (start 111.506 33.401) (end 112.395 34.29) (width 0.8) (layer B.Cu) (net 3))
 (segment (start 111.506 31.242) (end 111.506 33.401) (width 0.8) (layer B.Cu) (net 3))
 (segment (start 118.745 34.29) (end 120.015 33.02) (width 0.8) (layer B.Cu) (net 3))
 (segment (start 120.015 33.02) (end 120.015 29.21) (width 0.8) (layer B.Cu) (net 3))
 (segment (start 112.395 34.29) (end 118.745 34.29) (width 0.8) (layer B.Cu) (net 3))
 (segment (start 83.566 31.242) (end 83.566 39.624) (width 0.8) (layer B.Cu) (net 14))
 (segment (start 75.525 45.3625) (end 81.32 45.3625) (width 0.8) (layer B.Cu) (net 14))
 (segment (start 83.566 43.1165) (end 83.566 39.624) (width 0.8) (layer B.Cu) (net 14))
 (segment (start 81.32 45.3625) (end 83.566 43.1165) (width 0.8) (layer B.Cu) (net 14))
 (segment (start 96.266 31.242) (end 96.266 31.642) (width 0.6) (layer B.Cu) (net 9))
 (segment (start 116.586 27.686) (end 116.586 31.242) (width 0.8) (layer B.Cu) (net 1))
 (segment (start 115.57 26.67) (end 116.586 27.686) (width 0.8) (layer B.Cu) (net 1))
 (segment (start 115.57 26.67) (end 112.15 26.67) (width 0.8) (layer B.Cu) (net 1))
 (segment (start 114.935 56.1975) (end 114.935 57.15) (width 0.5) (layer B.Cu) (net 27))
 (segment (start 115.8875 55.245) (end 114.935 56.1975) (width 0.5) (layer B.Cu) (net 27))
 (segment (start 115.8875 52.105) (end 115.8875 55.245) (width 0.5) (layer B.Cu) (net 27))
 (segment (start 114.6175 54.2925) (end 114.6175 52.105) (width 0.5) (layer B.Cu) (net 28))
 (segment (start 114.6175 54.9275) (end 114.6175 54.2925) (width 0.5) (layer B.Cu) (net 28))
 (segment (start 113.9825 55.5625) (end 114.6175 54.9275) (width 0.5) (layer B.Cu) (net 28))
 (segment (start 112.395 56.515) (end 113.3475 55.5625) (width 0.5) (layer B.Cu) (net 28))
 (segment (start 113.3475 55.5625) (end 113.9825 55.5625) (width 0.5) (layer B.Cu) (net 28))
 (segment (start 112.395 57.15) (end 112.395 56.515) (width 0.5) (layer B.Cu) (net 28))
 (segment (start 113.3475 52.105) (end 113.3475 54.2925) (width 0.5) (layer B.Cu) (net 29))
 (segment (start 113.3475 54.2925) (end 112.7125 54.9275) (width 0.5) (layer B.Cu) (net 29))
 (segment (start 112.7125 54.9275) (end 112.0775 54.9275) (width 0.5) (layer B.Cu) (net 29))
 (segment (start 112.0775 54.9275) (end 109.855 57.15) (width 0.5) (layer B.Cu) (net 29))
 (segment (start 112.0775 53.6575) (end 112.0775 52.105) (width 0.5) (layer B.Cu) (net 30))
 (segment (start 110.8075 53.6575) (end 112.0775 53.6575) (width 0.5) (layer B.Cu) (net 30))
 (segment (start 107.315 57.15) (end 110.8075 53.6575) (width 0.5) (layer B.Cu) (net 30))
 (segment (start 115.8875 46.955) (end 118.4275 46.955) (width 0.5) (layer B.Cu) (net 31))
 (segment (start 119.77 49.6025) (end 122.2375 49.6025) (width 0.5) (layer B.Cu) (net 31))
 (segment (start 118.4275 48.26) (end 119.77 49.6025) (width 0.5) (layer B.Cu) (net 31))
 (segment (start 118.4275 46.955) (end 118.4275 48.26) (width 0.5) (layer B.Cu) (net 31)))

